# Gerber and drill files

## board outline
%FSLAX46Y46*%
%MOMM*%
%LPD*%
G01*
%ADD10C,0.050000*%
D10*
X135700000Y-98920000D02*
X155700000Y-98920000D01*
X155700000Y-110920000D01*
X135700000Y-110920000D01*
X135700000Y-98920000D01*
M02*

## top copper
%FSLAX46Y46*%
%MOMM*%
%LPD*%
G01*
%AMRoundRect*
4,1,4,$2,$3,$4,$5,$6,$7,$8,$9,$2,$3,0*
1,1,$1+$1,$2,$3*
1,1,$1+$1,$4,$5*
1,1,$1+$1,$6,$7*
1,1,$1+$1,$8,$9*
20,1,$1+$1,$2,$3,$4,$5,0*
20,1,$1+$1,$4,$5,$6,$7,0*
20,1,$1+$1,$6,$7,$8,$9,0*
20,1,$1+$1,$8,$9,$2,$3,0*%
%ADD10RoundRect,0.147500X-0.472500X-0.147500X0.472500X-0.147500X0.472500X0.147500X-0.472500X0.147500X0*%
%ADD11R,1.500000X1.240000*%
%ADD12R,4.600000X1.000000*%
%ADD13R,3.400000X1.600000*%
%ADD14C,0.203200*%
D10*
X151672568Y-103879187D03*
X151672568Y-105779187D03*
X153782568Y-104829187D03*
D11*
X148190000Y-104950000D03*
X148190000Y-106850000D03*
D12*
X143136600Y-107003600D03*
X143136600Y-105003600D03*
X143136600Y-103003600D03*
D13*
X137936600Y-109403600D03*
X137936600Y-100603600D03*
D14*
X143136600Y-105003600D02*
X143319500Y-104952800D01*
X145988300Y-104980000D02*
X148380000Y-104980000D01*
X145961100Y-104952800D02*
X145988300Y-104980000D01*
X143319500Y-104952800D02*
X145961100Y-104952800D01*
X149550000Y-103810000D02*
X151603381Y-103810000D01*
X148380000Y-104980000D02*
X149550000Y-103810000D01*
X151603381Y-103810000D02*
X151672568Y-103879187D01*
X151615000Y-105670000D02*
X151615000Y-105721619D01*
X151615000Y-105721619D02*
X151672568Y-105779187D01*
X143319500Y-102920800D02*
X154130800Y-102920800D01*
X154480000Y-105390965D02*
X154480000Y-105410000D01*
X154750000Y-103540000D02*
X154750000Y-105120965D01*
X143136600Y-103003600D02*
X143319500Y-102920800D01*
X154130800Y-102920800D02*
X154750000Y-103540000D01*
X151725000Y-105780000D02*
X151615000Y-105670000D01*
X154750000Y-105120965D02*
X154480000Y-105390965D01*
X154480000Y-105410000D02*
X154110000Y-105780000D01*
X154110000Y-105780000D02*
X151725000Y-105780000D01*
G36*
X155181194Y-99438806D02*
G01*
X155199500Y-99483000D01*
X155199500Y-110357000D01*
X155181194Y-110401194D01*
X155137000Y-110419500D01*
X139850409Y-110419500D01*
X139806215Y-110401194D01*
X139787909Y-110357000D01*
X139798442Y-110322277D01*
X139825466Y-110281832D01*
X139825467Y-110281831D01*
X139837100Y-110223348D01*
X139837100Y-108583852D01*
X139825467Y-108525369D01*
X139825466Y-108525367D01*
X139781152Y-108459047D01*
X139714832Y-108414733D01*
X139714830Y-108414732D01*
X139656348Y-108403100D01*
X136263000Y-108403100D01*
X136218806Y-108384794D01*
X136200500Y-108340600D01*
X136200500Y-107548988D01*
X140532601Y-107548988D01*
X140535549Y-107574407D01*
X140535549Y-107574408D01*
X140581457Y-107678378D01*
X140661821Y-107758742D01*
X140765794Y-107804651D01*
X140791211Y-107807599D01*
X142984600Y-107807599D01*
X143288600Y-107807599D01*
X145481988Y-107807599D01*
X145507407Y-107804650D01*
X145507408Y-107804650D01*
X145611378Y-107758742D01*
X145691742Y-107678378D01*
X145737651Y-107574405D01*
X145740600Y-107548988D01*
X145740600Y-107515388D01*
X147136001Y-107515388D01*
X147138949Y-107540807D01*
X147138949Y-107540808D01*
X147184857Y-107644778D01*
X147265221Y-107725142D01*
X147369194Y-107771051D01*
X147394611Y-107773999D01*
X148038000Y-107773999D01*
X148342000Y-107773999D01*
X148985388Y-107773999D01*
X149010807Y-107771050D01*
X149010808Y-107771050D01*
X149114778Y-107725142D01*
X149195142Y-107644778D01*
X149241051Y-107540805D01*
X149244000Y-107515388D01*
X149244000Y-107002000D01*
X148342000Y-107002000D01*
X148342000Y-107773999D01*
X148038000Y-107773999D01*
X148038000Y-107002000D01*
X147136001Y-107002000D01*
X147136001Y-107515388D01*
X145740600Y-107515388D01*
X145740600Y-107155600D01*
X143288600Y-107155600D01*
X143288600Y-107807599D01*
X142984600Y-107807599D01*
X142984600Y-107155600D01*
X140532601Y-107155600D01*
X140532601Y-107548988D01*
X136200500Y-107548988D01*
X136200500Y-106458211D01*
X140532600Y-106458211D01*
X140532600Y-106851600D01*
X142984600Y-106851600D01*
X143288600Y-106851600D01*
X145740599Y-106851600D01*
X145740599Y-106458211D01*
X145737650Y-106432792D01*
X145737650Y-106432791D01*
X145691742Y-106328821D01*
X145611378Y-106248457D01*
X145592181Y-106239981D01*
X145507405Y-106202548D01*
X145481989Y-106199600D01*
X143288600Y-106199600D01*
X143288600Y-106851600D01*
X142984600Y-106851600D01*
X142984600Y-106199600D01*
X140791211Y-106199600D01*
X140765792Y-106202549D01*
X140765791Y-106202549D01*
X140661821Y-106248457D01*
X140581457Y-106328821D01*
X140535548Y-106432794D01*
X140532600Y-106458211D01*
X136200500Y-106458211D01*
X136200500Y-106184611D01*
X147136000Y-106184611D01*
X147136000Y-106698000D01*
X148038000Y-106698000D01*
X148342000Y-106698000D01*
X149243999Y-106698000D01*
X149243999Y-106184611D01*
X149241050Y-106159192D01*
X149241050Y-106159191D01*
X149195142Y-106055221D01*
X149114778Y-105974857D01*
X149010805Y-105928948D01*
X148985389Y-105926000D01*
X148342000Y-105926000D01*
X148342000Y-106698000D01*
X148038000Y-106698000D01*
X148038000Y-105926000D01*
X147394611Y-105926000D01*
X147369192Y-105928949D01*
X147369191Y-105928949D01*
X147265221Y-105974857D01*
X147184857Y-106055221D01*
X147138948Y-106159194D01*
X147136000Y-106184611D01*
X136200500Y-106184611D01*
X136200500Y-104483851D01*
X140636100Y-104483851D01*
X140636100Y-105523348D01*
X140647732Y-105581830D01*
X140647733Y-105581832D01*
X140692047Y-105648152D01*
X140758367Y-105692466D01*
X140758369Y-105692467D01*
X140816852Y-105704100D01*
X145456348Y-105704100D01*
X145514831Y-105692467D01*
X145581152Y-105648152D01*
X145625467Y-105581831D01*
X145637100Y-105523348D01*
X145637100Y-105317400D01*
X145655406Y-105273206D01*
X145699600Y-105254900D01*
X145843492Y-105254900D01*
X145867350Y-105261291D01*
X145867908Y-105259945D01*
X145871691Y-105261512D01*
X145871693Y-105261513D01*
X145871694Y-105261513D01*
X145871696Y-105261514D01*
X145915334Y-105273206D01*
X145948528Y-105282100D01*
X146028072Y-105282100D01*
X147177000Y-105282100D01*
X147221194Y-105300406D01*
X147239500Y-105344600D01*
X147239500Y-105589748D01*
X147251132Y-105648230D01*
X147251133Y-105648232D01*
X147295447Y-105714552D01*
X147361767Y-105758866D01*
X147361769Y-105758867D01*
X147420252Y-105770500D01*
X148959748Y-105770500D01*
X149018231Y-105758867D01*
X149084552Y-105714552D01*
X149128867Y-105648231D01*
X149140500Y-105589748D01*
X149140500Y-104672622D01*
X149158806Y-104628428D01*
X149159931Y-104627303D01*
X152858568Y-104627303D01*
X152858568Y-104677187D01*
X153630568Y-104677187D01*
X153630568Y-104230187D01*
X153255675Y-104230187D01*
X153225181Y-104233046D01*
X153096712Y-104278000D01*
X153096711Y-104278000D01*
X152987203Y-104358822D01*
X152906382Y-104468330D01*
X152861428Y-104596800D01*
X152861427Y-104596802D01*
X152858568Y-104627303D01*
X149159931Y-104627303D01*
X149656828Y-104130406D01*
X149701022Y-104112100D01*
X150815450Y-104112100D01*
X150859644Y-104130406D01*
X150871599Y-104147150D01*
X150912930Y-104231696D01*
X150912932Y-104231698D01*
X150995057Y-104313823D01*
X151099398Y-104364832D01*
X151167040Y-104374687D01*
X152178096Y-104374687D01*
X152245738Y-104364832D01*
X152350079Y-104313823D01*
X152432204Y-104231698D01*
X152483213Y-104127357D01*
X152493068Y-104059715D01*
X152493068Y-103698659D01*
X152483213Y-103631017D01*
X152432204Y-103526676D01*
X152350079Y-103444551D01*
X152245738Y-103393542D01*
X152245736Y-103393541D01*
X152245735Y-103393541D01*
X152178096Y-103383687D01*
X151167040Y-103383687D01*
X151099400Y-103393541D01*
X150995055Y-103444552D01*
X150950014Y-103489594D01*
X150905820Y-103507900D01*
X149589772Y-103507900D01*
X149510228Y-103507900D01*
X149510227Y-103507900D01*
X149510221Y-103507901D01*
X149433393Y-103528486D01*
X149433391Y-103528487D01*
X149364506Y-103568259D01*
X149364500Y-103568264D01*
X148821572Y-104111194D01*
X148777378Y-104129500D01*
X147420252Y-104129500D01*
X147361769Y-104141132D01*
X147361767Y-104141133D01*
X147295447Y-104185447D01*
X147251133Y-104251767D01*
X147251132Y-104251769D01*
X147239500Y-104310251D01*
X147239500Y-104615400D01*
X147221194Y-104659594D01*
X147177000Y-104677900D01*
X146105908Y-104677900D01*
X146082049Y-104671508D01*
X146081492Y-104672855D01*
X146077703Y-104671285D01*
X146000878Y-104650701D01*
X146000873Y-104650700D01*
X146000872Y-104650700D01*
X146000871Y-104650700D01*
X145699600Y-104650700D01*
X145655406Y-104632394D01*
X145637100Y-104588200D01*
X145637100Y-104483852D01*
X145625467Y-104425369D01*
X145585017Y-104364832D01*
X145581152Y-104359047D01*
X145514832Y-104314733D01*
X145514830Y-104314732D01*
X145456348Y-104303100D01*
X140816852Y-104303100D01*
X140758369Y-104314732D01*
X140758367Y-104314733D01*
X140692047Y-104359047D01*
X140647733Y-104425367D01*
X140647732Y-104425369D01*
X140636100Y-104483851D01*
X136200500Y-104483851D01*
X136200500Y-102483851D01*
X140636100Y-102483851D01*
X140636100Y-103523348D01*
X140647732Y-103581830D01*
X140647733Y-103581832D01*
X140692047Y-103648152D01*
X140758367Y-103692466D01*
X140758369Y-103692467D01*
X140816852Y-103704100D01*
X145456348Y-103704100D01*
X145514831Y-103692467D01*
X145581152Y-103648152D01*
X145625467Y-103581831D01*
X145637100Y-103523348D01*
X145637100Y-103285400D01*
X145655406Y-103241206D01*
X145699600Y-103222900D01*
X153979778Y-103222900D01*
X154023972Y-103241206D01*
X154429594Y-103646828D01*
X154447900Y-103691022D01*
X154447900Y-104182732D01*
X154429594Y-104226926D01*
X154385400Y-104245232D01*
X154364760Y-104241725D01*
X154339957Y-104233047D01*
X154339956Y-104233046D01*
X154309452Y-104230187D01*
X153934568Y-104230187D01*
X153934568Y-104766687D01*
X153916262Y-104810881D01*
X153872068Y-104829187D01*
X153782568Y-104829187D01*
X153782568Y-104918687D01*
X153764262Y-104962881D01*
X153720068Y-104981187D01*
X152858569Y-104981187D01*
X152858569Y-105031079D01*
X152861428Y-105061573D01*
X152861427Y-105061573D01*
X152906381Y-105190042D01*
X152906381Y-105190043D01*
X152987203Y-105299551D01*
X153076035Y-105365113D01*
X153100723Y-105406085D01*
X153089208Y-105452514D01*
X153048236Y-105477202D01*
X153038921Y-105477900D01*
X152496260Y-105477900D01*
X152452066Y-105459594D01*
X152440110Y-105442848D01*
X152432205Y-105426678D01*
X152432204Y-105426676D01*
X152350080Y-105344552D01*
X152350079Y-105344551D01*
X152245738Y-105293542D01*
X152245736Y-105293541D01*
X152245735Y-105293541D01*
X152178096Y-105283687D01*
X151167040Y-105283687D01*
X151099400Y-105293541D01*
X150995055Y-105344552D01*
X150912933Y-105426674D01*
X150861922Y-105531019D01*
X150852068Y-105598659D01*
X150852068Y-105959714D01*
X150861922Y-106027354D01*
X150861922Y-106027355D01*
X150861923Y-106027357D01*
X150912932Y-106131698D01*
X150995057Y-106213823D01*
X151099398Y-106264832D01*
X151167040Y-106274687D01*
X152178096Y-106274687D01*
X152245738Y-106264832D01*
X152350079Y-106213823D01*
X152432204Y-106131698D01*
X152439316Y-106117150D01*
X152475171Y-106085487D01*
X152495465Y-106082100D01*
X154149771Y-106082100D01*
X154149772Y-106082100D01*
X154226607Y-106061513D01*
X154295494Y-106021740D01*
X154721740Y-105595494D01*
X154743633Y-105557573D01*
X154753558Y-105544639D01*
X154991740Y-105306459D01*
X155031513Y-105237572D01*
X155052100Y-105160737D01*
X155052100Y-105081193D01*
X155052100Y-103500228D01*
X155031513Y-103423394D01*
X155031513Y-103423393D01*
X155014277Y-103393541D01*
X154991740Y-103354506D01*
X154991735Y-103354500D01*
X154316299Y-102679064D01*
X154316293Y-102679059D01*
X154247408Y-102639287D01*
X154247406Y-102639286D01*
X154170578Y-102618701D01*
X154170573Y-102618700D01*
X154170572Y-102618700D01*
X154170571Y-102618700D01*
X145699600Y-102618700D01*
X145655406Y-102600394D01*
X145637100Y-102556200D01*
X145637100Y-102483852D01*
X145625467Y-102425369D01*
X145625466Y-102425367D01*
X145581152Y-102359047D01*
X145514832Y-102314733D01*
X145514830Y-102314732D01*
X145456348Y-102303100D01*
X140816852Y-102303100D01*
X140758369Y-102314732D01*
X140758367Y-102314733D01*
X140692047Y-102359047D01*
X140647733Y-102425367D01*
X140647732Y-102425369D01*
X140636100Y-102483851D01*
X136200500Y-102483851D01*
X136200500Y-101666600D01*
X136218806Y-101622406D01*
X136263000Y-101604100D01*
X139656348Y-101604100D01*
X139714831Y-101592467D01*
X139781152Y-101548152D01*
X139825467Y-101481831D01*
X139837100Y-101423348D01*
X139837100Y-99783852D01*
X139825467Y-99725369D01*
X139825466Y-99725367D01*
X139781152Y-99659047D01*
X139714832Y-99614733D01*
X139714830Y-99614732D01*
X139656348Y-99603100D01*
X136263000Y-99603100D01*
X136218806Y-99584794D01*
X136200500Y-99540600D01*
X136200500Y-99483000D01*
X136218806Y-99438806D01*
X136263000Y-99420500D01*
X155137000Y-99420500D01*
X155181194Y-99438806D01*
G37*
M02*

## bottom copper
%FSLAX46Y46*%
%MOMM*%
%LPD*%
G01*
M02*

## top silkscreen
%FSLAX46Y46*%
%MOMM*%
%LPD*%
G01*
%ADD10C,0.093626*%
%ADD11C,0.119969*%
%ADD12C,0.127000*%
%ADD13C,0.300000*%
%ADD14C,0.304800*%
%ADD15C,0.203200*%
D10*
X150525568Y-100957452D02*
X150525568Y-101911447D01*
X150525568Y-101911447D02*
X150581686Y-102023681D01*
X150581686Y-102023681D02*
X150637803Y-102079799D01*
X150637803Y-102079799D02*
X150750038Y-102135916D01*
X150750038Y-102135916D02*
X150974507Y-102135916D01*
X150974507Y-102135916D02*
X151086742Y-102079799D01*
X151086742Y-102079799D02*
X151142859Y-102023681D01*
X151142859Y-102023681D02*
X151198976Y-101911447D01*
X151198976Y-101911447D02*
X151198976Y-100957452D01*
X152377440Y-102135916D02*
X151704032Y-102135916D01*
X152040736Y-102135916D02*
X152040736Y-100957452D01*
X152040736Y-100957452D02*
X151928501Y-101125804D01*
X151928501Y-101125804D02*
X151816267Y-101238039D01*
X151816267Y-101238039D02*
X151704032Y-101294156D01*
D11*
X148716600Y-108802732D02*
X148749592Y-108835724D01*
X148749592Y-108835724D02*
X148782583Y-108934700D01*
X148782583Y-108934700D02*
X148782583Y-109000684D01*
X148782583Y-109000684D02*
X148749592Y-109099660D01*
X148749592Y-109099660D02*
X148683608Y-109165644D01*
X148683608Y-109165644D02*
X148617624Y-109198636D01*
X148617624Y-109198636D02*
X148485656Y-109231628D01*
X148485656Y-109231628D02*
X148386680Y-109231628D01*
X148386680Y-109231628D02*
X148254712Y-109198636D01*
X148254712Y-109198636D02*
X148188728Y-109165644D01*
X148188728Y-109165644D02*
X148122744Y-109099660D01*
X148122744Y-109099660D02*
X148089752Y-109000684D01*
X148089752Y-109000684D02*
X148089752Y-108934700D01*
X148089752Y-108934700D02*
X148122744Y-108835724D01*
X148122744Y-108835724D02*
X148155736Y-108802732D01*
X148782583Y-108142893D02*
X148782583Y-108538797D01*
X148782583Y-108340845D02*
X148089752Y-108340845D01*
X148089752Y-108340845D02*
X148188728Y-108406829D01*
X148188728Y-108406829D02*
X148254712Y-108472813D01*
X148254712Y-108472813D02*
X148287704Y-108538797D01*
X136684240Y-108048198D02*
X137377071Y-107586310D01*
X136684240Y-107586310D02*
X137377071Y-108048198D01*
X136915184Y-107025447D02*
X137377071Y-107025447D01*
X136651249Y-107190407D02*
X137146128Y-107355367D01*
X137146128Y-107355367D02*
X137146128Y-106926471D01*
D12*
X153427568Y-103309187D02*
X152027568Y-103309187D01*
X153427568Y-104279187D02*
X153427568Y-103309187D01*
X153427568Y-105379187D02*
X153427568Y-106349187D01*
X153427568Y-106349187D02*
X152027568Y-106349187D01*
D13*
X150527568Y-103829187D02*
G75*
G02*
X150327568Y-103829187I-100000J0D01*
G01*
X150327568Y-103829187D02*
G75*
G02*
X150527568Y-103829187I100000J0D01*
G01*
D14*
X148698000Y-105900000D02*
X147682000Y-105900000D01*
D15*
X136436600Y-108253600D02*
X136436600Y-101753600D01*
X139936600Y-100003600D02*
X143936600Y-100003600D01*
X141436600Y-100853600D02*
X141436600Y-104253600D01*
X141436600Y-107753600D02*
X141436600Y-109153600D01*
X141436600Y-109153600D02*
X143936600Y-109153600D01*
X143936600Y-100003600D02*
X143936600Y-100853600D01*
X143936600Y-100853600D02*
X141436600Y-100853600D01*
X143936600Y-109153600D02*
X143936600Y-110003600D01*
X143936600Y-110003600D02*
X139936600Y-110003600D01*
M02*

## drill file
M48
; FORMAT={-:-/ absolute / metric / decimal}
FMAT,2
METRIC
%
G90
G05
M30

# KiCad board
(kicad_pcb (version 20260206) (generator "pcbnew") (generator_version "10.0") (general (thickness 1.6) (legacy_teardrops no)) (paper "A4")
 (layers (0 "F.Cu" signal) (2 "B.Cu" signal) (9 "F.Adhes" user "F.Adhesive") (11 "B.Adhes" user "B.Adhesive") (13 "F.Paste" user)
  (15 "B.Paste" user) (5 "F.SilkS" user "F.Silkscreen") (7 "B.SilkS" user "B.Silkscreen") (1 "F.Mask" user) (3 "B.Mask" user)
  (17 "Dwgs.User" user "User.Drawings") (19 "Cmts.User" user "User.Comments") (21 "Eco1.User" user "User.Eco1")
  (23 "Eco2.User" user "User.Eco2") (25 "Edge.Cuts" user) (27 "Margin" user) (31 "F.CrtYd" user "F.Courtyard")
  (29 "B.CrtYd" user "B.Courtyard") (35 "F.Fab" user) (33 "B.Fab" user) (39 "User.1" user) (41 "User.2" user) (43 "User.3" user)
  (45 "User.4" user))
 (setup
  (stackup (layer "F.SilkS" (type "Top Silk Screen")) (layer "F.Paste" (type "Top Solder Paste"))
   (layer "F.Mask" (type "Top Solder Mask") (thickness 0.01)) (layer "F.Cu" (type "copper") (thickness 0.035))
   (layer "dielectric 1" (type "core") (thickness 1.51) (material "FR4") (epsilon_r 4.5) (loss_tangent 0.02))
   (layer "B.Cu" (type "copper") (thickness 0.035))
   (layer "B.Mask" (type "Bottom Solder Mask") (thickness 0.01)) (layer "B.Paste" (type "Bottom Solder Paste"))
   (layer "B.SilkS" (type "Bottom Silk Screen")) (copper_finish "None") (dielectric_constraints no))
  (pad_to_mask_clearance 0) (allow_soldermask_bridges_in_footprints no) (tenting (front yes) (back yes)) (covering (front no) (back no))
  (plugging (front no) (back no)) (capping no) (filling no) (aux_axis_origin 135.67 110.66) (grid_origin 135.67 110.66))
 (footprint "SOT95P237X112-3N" (layer "F.Cu") (at 152.727568 104.829187)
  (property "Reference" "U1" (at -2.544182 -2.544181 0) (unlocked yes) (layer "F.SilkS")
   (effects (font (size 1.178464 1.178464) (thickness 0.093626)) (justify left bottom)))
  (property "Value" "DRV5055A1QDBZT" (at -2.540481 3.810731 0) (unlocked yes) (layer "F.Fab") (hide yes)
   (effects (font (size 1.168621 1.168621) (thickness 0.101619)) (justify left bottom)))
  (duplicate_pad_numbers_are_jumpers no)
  (fp_line (start 0.7 -1.52) (end -0.7 -1.52) (stroke (width 0.127) (type solid)) (layer "F.SilkS"))
  (fp_line (start 0.7 -0.55) (end 0.7 -1.52) (stroke (width 0.127) (type solid)) (layer "F.SilkS"))
  (fp_line (start 0.7 0.55) (end 0.7 1.52) (stroke (width 0.127) (type solid)) (layer "F.SilkS"))
  (fp_line (start 0.7 1.52) (end -0.7 1.52) (stroke (width 0.127) (type solid)) (layer "F.SilkS"))
  (fp_circle (center -2.3 -1) (end -2.2 -1) (stroke (width 0.3) (type solid)) (fill no) (layer "F.SilkS"))
  (pad "1" smd roundrect (at -1.055 -0.95) (size 1.24 0.59) (layers "F.Cu" "F.Mask" "F.Paste") (roundrect_rratio 0.25) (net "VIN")
   (solder_mask_margin 0.0635) (solder_paste_margin 0) (thermal_bridge_angle 0))
  (pad "2" smd roundrect (at -1.055 0.95) (size 1.24 0.59) (layers "F.Cu" "F.Mask" "F.Paste") (roundrect_rratio 0.25) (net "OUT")
   (solder_mask_margin 0.0635) (solder_paste_margin 0) (thermal_bridge_angle 0))
  (pad "3" smd roundrect (at 1.055 0) (size 1.24 0.59) (layers "F.Cu" "F.Mask" "F.Paste") (roundrect_rratio 0.25) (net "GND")
   (solder_mask_margin 0.0635) (solder_paste_margin 0) (thermal_bridge_angle 0)))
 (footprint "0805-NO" (layer "F.Cu") (at 148.19 105.9 -90)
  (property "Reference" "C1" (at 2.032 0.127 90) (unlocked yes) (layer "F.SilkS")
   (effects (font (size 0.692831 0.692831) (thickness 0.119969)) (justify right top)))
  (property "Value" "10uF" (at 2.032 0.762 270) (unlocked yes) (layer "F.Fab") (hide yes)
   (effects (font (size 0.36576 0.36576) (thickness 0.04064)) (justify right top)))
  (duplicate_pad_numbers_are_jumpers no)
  (fp_line (start 0 -0.508) (end 0 0.508) (stroke (width 0.3048) (type solid)) (layer "F.SilkS"))
  (pad "1" smd rect (at -0.95 0 270) (size 1.24 1.5) (layers "F.Cu" "F.Mask" "F.Paste") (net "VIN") (solder_mask_margin 0.0635)
   (solder_paste_margin 0) (thermal_bridge_angle 0))
  (pad "2" smd rect (at 0.95 0 270) (size 1.24 1.5) (layers "F.Cu" "F.Mask" "F.Paste") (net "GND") (solder_mask_margin 0.0635)
   (solder_paste_margin 0) (thermal_bridge_angle 0)))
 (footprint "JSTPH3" (layer "F.Cu") (at 140.4366 105.0036 90)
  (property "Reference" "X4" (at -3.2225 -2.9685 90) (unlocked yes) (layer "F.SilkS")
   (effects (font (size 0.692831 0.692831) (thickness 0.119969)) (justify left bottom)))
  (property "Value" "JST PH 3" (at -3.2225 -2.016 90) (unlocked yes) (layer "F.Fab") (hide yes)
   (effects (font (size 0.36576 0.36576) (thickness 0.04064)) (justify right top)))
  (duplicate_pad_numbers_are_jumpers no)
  (fp_line (start -3.25 -4) (end 3.25 -4) (stroke (width 0.2032) (type solid)) (layer "F.SilkS"))
  (fp_line (start 5 -0.5) (end 5 3.5) (stroke (width 0.2032) (type solid)) (layer "F.SilkS"))
  (fp_line (start 4.15 1) (end 0.75 1) (stroke (width 0.2032) (type solid)) (layer "F.SilkS"))
  (fp_line (start -2.75 1) (end -4.15 1) (stroke (width 0.2032) (type solid)) (layer "F.SilkS"))
  (fp_line (start -4.15 1) (end -4.15 3.5) (stroke (width 0.2032) (type solid)) (layer "F.SilkS"))
  (fp_line (start 5 3.5) (end 4.15 3.5) (stroke (width 0.2032) (type solid)) (layer "F.SilkS"))
  (fp_line (start 4.15 3.5) (end 4.15 1) (stroke (width 0.2032) (type solid)) (layer "F.SilkS"))
  (fp_line (start -4.15 3.5) (end -5 3.5) (stroke (width 0.2032) (type solid)) (layer "F.SilkS"))
  (fp_line (start -5 3.5) (end -5 -0.5) (stroke (width 0.2032) (type solid)) (layer "F.SilkS"))
  (pad "1" smd rect (at -2 2.7 90) (size 1 4.6) (layers "F.Cu" "F.Mask" "F.Paste") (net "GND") (solder_mask_margin 0.0635)
   (solder_paste_margin 0) (thermal_bridge_angle 0))
  (pad "2" smd rect (at 0 2.7 90) (size 1 4.6) (layers "F.Cu" "F.Mask" "F.Paste") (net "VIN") (solder_mask_margin 0.0635)
   (solder_paste_margin 0) (thermal_bridge_angle 0))
  (pad "3" smd rect (at 2 2.7 90) (size 1 4.6) (layers "F.Cu" "F.Mask" "F.Paste") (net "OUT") (solder_mask_margin 0.0635)
   (solder_paste_margin 0) (thermal_bridge_angle 0))
  (pad "NC1" smd rect (at -4.4 -2.5 180) (size 3.4 1.6) (layers "F.Cu" "F.Mask" "F.Paste") (solder_mask_margin 0.0635)
   (solder_paste_margin 0) (thermal_bridge_angle 0))
  (pad "NC2" smd rect (at 4.4 -2.5 180) (size 3.4 1.6) (layers "F.Cu" "F.Mask" "F.Paste") (solder_mask_margin 0.0635)
   (solder_paste_margin 0) (thermal_bridge_angle 0)))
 (gr_rect (start 135.7 98.92) (end 155.7 110.92) (stroke (width 0.05) (type solid)) (fill no) (layer "Edge.Cuts"))
 (segment (start 143.1366 105.0036) (end 143.3195 104.9528) (width 0.2032) (layer "F.Cu") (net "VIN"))
 (segment (start 145.9883 104.98) (end 148.38 104.98) (width 0.2032) (layer "F.Cu") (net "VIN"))
 (segment (start 145.9611 104.9528) (end 145.9883 104.98) (width 0.2032) (layer "F.Cu") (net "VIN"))
 (segment (start 143.3195 104.9528) (end 145.9611 104.9528) (width 0.2032) (layer "F.Cu") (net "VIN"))
 (segment (start 149.55 103.81) (end 151.603381 103.81) (width 0.2032) (layer "F.Cu") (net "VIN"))
 (segment (start 148.38 104.98) (end 149.55 103.81) (width 0.2032) (layer "F.Cu") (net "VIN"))
 (segment (start 151.603381 103.81) (end 151.672568 103.879187) (width 0.2032) (layer "F.Cu") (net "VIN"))
 (segment (start 151.615 105.67) (end 151.615 105.721619) (width 0.2032) (layer "F.Cu") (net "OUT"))
 (segment (start 151.615 105.721619) (end 151.672568 105.779187) (width 0.2032) (layer "F.Cu") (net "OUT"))
 (segment (start 143.3195 102.9208) (end 154.1308 102.9208) (width 0.2032) (layer "F.Cu") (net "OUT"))
 (segment (start 154.48 105.390965) (end 154.48 105.41) (width 0.2032) (layer "F.Cu") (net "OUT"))
 (segment (start 154.75 103.54) (end 154.75 105.120965) (width 0.2032) (layer "F.Cu") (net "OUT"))
 (segment (start 143.1366 103.0036) (end 143.3195 102.9208) (width 0.2032) (layer "F.Cu") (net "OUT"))
 (segment (start 154.1308 102.9208) (end 154.75 103.54) (width 0.2032) (layer "F.Cu") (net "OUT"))
 (segment (start 151.725 105.78) (end 151.615 105.67) (width 0.2032) (layer "F.Cu") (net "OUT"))
 (segment (start 154.75 105.120965) (end 154.48 105.390965) (width 0.2032) (layer "F.Cu") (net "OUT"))
 (segment (start 154.48 105.41) (end 154.11 105.78) (width 0.2032) (layer "F.Cu") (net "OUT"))
 (segment (start 154.11 105.78) (end 151.725 105.78) (width 0.2032) (layer "F.Cu") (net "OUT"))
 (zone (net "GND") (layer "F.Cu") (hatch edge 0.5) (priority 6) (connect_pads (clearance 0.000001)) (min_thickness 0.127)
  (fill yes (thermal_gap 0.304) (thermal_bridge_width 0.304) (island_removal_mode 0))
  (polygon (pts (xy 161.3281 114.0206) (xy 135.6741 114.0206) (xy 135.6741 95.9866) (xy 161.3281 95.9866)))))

